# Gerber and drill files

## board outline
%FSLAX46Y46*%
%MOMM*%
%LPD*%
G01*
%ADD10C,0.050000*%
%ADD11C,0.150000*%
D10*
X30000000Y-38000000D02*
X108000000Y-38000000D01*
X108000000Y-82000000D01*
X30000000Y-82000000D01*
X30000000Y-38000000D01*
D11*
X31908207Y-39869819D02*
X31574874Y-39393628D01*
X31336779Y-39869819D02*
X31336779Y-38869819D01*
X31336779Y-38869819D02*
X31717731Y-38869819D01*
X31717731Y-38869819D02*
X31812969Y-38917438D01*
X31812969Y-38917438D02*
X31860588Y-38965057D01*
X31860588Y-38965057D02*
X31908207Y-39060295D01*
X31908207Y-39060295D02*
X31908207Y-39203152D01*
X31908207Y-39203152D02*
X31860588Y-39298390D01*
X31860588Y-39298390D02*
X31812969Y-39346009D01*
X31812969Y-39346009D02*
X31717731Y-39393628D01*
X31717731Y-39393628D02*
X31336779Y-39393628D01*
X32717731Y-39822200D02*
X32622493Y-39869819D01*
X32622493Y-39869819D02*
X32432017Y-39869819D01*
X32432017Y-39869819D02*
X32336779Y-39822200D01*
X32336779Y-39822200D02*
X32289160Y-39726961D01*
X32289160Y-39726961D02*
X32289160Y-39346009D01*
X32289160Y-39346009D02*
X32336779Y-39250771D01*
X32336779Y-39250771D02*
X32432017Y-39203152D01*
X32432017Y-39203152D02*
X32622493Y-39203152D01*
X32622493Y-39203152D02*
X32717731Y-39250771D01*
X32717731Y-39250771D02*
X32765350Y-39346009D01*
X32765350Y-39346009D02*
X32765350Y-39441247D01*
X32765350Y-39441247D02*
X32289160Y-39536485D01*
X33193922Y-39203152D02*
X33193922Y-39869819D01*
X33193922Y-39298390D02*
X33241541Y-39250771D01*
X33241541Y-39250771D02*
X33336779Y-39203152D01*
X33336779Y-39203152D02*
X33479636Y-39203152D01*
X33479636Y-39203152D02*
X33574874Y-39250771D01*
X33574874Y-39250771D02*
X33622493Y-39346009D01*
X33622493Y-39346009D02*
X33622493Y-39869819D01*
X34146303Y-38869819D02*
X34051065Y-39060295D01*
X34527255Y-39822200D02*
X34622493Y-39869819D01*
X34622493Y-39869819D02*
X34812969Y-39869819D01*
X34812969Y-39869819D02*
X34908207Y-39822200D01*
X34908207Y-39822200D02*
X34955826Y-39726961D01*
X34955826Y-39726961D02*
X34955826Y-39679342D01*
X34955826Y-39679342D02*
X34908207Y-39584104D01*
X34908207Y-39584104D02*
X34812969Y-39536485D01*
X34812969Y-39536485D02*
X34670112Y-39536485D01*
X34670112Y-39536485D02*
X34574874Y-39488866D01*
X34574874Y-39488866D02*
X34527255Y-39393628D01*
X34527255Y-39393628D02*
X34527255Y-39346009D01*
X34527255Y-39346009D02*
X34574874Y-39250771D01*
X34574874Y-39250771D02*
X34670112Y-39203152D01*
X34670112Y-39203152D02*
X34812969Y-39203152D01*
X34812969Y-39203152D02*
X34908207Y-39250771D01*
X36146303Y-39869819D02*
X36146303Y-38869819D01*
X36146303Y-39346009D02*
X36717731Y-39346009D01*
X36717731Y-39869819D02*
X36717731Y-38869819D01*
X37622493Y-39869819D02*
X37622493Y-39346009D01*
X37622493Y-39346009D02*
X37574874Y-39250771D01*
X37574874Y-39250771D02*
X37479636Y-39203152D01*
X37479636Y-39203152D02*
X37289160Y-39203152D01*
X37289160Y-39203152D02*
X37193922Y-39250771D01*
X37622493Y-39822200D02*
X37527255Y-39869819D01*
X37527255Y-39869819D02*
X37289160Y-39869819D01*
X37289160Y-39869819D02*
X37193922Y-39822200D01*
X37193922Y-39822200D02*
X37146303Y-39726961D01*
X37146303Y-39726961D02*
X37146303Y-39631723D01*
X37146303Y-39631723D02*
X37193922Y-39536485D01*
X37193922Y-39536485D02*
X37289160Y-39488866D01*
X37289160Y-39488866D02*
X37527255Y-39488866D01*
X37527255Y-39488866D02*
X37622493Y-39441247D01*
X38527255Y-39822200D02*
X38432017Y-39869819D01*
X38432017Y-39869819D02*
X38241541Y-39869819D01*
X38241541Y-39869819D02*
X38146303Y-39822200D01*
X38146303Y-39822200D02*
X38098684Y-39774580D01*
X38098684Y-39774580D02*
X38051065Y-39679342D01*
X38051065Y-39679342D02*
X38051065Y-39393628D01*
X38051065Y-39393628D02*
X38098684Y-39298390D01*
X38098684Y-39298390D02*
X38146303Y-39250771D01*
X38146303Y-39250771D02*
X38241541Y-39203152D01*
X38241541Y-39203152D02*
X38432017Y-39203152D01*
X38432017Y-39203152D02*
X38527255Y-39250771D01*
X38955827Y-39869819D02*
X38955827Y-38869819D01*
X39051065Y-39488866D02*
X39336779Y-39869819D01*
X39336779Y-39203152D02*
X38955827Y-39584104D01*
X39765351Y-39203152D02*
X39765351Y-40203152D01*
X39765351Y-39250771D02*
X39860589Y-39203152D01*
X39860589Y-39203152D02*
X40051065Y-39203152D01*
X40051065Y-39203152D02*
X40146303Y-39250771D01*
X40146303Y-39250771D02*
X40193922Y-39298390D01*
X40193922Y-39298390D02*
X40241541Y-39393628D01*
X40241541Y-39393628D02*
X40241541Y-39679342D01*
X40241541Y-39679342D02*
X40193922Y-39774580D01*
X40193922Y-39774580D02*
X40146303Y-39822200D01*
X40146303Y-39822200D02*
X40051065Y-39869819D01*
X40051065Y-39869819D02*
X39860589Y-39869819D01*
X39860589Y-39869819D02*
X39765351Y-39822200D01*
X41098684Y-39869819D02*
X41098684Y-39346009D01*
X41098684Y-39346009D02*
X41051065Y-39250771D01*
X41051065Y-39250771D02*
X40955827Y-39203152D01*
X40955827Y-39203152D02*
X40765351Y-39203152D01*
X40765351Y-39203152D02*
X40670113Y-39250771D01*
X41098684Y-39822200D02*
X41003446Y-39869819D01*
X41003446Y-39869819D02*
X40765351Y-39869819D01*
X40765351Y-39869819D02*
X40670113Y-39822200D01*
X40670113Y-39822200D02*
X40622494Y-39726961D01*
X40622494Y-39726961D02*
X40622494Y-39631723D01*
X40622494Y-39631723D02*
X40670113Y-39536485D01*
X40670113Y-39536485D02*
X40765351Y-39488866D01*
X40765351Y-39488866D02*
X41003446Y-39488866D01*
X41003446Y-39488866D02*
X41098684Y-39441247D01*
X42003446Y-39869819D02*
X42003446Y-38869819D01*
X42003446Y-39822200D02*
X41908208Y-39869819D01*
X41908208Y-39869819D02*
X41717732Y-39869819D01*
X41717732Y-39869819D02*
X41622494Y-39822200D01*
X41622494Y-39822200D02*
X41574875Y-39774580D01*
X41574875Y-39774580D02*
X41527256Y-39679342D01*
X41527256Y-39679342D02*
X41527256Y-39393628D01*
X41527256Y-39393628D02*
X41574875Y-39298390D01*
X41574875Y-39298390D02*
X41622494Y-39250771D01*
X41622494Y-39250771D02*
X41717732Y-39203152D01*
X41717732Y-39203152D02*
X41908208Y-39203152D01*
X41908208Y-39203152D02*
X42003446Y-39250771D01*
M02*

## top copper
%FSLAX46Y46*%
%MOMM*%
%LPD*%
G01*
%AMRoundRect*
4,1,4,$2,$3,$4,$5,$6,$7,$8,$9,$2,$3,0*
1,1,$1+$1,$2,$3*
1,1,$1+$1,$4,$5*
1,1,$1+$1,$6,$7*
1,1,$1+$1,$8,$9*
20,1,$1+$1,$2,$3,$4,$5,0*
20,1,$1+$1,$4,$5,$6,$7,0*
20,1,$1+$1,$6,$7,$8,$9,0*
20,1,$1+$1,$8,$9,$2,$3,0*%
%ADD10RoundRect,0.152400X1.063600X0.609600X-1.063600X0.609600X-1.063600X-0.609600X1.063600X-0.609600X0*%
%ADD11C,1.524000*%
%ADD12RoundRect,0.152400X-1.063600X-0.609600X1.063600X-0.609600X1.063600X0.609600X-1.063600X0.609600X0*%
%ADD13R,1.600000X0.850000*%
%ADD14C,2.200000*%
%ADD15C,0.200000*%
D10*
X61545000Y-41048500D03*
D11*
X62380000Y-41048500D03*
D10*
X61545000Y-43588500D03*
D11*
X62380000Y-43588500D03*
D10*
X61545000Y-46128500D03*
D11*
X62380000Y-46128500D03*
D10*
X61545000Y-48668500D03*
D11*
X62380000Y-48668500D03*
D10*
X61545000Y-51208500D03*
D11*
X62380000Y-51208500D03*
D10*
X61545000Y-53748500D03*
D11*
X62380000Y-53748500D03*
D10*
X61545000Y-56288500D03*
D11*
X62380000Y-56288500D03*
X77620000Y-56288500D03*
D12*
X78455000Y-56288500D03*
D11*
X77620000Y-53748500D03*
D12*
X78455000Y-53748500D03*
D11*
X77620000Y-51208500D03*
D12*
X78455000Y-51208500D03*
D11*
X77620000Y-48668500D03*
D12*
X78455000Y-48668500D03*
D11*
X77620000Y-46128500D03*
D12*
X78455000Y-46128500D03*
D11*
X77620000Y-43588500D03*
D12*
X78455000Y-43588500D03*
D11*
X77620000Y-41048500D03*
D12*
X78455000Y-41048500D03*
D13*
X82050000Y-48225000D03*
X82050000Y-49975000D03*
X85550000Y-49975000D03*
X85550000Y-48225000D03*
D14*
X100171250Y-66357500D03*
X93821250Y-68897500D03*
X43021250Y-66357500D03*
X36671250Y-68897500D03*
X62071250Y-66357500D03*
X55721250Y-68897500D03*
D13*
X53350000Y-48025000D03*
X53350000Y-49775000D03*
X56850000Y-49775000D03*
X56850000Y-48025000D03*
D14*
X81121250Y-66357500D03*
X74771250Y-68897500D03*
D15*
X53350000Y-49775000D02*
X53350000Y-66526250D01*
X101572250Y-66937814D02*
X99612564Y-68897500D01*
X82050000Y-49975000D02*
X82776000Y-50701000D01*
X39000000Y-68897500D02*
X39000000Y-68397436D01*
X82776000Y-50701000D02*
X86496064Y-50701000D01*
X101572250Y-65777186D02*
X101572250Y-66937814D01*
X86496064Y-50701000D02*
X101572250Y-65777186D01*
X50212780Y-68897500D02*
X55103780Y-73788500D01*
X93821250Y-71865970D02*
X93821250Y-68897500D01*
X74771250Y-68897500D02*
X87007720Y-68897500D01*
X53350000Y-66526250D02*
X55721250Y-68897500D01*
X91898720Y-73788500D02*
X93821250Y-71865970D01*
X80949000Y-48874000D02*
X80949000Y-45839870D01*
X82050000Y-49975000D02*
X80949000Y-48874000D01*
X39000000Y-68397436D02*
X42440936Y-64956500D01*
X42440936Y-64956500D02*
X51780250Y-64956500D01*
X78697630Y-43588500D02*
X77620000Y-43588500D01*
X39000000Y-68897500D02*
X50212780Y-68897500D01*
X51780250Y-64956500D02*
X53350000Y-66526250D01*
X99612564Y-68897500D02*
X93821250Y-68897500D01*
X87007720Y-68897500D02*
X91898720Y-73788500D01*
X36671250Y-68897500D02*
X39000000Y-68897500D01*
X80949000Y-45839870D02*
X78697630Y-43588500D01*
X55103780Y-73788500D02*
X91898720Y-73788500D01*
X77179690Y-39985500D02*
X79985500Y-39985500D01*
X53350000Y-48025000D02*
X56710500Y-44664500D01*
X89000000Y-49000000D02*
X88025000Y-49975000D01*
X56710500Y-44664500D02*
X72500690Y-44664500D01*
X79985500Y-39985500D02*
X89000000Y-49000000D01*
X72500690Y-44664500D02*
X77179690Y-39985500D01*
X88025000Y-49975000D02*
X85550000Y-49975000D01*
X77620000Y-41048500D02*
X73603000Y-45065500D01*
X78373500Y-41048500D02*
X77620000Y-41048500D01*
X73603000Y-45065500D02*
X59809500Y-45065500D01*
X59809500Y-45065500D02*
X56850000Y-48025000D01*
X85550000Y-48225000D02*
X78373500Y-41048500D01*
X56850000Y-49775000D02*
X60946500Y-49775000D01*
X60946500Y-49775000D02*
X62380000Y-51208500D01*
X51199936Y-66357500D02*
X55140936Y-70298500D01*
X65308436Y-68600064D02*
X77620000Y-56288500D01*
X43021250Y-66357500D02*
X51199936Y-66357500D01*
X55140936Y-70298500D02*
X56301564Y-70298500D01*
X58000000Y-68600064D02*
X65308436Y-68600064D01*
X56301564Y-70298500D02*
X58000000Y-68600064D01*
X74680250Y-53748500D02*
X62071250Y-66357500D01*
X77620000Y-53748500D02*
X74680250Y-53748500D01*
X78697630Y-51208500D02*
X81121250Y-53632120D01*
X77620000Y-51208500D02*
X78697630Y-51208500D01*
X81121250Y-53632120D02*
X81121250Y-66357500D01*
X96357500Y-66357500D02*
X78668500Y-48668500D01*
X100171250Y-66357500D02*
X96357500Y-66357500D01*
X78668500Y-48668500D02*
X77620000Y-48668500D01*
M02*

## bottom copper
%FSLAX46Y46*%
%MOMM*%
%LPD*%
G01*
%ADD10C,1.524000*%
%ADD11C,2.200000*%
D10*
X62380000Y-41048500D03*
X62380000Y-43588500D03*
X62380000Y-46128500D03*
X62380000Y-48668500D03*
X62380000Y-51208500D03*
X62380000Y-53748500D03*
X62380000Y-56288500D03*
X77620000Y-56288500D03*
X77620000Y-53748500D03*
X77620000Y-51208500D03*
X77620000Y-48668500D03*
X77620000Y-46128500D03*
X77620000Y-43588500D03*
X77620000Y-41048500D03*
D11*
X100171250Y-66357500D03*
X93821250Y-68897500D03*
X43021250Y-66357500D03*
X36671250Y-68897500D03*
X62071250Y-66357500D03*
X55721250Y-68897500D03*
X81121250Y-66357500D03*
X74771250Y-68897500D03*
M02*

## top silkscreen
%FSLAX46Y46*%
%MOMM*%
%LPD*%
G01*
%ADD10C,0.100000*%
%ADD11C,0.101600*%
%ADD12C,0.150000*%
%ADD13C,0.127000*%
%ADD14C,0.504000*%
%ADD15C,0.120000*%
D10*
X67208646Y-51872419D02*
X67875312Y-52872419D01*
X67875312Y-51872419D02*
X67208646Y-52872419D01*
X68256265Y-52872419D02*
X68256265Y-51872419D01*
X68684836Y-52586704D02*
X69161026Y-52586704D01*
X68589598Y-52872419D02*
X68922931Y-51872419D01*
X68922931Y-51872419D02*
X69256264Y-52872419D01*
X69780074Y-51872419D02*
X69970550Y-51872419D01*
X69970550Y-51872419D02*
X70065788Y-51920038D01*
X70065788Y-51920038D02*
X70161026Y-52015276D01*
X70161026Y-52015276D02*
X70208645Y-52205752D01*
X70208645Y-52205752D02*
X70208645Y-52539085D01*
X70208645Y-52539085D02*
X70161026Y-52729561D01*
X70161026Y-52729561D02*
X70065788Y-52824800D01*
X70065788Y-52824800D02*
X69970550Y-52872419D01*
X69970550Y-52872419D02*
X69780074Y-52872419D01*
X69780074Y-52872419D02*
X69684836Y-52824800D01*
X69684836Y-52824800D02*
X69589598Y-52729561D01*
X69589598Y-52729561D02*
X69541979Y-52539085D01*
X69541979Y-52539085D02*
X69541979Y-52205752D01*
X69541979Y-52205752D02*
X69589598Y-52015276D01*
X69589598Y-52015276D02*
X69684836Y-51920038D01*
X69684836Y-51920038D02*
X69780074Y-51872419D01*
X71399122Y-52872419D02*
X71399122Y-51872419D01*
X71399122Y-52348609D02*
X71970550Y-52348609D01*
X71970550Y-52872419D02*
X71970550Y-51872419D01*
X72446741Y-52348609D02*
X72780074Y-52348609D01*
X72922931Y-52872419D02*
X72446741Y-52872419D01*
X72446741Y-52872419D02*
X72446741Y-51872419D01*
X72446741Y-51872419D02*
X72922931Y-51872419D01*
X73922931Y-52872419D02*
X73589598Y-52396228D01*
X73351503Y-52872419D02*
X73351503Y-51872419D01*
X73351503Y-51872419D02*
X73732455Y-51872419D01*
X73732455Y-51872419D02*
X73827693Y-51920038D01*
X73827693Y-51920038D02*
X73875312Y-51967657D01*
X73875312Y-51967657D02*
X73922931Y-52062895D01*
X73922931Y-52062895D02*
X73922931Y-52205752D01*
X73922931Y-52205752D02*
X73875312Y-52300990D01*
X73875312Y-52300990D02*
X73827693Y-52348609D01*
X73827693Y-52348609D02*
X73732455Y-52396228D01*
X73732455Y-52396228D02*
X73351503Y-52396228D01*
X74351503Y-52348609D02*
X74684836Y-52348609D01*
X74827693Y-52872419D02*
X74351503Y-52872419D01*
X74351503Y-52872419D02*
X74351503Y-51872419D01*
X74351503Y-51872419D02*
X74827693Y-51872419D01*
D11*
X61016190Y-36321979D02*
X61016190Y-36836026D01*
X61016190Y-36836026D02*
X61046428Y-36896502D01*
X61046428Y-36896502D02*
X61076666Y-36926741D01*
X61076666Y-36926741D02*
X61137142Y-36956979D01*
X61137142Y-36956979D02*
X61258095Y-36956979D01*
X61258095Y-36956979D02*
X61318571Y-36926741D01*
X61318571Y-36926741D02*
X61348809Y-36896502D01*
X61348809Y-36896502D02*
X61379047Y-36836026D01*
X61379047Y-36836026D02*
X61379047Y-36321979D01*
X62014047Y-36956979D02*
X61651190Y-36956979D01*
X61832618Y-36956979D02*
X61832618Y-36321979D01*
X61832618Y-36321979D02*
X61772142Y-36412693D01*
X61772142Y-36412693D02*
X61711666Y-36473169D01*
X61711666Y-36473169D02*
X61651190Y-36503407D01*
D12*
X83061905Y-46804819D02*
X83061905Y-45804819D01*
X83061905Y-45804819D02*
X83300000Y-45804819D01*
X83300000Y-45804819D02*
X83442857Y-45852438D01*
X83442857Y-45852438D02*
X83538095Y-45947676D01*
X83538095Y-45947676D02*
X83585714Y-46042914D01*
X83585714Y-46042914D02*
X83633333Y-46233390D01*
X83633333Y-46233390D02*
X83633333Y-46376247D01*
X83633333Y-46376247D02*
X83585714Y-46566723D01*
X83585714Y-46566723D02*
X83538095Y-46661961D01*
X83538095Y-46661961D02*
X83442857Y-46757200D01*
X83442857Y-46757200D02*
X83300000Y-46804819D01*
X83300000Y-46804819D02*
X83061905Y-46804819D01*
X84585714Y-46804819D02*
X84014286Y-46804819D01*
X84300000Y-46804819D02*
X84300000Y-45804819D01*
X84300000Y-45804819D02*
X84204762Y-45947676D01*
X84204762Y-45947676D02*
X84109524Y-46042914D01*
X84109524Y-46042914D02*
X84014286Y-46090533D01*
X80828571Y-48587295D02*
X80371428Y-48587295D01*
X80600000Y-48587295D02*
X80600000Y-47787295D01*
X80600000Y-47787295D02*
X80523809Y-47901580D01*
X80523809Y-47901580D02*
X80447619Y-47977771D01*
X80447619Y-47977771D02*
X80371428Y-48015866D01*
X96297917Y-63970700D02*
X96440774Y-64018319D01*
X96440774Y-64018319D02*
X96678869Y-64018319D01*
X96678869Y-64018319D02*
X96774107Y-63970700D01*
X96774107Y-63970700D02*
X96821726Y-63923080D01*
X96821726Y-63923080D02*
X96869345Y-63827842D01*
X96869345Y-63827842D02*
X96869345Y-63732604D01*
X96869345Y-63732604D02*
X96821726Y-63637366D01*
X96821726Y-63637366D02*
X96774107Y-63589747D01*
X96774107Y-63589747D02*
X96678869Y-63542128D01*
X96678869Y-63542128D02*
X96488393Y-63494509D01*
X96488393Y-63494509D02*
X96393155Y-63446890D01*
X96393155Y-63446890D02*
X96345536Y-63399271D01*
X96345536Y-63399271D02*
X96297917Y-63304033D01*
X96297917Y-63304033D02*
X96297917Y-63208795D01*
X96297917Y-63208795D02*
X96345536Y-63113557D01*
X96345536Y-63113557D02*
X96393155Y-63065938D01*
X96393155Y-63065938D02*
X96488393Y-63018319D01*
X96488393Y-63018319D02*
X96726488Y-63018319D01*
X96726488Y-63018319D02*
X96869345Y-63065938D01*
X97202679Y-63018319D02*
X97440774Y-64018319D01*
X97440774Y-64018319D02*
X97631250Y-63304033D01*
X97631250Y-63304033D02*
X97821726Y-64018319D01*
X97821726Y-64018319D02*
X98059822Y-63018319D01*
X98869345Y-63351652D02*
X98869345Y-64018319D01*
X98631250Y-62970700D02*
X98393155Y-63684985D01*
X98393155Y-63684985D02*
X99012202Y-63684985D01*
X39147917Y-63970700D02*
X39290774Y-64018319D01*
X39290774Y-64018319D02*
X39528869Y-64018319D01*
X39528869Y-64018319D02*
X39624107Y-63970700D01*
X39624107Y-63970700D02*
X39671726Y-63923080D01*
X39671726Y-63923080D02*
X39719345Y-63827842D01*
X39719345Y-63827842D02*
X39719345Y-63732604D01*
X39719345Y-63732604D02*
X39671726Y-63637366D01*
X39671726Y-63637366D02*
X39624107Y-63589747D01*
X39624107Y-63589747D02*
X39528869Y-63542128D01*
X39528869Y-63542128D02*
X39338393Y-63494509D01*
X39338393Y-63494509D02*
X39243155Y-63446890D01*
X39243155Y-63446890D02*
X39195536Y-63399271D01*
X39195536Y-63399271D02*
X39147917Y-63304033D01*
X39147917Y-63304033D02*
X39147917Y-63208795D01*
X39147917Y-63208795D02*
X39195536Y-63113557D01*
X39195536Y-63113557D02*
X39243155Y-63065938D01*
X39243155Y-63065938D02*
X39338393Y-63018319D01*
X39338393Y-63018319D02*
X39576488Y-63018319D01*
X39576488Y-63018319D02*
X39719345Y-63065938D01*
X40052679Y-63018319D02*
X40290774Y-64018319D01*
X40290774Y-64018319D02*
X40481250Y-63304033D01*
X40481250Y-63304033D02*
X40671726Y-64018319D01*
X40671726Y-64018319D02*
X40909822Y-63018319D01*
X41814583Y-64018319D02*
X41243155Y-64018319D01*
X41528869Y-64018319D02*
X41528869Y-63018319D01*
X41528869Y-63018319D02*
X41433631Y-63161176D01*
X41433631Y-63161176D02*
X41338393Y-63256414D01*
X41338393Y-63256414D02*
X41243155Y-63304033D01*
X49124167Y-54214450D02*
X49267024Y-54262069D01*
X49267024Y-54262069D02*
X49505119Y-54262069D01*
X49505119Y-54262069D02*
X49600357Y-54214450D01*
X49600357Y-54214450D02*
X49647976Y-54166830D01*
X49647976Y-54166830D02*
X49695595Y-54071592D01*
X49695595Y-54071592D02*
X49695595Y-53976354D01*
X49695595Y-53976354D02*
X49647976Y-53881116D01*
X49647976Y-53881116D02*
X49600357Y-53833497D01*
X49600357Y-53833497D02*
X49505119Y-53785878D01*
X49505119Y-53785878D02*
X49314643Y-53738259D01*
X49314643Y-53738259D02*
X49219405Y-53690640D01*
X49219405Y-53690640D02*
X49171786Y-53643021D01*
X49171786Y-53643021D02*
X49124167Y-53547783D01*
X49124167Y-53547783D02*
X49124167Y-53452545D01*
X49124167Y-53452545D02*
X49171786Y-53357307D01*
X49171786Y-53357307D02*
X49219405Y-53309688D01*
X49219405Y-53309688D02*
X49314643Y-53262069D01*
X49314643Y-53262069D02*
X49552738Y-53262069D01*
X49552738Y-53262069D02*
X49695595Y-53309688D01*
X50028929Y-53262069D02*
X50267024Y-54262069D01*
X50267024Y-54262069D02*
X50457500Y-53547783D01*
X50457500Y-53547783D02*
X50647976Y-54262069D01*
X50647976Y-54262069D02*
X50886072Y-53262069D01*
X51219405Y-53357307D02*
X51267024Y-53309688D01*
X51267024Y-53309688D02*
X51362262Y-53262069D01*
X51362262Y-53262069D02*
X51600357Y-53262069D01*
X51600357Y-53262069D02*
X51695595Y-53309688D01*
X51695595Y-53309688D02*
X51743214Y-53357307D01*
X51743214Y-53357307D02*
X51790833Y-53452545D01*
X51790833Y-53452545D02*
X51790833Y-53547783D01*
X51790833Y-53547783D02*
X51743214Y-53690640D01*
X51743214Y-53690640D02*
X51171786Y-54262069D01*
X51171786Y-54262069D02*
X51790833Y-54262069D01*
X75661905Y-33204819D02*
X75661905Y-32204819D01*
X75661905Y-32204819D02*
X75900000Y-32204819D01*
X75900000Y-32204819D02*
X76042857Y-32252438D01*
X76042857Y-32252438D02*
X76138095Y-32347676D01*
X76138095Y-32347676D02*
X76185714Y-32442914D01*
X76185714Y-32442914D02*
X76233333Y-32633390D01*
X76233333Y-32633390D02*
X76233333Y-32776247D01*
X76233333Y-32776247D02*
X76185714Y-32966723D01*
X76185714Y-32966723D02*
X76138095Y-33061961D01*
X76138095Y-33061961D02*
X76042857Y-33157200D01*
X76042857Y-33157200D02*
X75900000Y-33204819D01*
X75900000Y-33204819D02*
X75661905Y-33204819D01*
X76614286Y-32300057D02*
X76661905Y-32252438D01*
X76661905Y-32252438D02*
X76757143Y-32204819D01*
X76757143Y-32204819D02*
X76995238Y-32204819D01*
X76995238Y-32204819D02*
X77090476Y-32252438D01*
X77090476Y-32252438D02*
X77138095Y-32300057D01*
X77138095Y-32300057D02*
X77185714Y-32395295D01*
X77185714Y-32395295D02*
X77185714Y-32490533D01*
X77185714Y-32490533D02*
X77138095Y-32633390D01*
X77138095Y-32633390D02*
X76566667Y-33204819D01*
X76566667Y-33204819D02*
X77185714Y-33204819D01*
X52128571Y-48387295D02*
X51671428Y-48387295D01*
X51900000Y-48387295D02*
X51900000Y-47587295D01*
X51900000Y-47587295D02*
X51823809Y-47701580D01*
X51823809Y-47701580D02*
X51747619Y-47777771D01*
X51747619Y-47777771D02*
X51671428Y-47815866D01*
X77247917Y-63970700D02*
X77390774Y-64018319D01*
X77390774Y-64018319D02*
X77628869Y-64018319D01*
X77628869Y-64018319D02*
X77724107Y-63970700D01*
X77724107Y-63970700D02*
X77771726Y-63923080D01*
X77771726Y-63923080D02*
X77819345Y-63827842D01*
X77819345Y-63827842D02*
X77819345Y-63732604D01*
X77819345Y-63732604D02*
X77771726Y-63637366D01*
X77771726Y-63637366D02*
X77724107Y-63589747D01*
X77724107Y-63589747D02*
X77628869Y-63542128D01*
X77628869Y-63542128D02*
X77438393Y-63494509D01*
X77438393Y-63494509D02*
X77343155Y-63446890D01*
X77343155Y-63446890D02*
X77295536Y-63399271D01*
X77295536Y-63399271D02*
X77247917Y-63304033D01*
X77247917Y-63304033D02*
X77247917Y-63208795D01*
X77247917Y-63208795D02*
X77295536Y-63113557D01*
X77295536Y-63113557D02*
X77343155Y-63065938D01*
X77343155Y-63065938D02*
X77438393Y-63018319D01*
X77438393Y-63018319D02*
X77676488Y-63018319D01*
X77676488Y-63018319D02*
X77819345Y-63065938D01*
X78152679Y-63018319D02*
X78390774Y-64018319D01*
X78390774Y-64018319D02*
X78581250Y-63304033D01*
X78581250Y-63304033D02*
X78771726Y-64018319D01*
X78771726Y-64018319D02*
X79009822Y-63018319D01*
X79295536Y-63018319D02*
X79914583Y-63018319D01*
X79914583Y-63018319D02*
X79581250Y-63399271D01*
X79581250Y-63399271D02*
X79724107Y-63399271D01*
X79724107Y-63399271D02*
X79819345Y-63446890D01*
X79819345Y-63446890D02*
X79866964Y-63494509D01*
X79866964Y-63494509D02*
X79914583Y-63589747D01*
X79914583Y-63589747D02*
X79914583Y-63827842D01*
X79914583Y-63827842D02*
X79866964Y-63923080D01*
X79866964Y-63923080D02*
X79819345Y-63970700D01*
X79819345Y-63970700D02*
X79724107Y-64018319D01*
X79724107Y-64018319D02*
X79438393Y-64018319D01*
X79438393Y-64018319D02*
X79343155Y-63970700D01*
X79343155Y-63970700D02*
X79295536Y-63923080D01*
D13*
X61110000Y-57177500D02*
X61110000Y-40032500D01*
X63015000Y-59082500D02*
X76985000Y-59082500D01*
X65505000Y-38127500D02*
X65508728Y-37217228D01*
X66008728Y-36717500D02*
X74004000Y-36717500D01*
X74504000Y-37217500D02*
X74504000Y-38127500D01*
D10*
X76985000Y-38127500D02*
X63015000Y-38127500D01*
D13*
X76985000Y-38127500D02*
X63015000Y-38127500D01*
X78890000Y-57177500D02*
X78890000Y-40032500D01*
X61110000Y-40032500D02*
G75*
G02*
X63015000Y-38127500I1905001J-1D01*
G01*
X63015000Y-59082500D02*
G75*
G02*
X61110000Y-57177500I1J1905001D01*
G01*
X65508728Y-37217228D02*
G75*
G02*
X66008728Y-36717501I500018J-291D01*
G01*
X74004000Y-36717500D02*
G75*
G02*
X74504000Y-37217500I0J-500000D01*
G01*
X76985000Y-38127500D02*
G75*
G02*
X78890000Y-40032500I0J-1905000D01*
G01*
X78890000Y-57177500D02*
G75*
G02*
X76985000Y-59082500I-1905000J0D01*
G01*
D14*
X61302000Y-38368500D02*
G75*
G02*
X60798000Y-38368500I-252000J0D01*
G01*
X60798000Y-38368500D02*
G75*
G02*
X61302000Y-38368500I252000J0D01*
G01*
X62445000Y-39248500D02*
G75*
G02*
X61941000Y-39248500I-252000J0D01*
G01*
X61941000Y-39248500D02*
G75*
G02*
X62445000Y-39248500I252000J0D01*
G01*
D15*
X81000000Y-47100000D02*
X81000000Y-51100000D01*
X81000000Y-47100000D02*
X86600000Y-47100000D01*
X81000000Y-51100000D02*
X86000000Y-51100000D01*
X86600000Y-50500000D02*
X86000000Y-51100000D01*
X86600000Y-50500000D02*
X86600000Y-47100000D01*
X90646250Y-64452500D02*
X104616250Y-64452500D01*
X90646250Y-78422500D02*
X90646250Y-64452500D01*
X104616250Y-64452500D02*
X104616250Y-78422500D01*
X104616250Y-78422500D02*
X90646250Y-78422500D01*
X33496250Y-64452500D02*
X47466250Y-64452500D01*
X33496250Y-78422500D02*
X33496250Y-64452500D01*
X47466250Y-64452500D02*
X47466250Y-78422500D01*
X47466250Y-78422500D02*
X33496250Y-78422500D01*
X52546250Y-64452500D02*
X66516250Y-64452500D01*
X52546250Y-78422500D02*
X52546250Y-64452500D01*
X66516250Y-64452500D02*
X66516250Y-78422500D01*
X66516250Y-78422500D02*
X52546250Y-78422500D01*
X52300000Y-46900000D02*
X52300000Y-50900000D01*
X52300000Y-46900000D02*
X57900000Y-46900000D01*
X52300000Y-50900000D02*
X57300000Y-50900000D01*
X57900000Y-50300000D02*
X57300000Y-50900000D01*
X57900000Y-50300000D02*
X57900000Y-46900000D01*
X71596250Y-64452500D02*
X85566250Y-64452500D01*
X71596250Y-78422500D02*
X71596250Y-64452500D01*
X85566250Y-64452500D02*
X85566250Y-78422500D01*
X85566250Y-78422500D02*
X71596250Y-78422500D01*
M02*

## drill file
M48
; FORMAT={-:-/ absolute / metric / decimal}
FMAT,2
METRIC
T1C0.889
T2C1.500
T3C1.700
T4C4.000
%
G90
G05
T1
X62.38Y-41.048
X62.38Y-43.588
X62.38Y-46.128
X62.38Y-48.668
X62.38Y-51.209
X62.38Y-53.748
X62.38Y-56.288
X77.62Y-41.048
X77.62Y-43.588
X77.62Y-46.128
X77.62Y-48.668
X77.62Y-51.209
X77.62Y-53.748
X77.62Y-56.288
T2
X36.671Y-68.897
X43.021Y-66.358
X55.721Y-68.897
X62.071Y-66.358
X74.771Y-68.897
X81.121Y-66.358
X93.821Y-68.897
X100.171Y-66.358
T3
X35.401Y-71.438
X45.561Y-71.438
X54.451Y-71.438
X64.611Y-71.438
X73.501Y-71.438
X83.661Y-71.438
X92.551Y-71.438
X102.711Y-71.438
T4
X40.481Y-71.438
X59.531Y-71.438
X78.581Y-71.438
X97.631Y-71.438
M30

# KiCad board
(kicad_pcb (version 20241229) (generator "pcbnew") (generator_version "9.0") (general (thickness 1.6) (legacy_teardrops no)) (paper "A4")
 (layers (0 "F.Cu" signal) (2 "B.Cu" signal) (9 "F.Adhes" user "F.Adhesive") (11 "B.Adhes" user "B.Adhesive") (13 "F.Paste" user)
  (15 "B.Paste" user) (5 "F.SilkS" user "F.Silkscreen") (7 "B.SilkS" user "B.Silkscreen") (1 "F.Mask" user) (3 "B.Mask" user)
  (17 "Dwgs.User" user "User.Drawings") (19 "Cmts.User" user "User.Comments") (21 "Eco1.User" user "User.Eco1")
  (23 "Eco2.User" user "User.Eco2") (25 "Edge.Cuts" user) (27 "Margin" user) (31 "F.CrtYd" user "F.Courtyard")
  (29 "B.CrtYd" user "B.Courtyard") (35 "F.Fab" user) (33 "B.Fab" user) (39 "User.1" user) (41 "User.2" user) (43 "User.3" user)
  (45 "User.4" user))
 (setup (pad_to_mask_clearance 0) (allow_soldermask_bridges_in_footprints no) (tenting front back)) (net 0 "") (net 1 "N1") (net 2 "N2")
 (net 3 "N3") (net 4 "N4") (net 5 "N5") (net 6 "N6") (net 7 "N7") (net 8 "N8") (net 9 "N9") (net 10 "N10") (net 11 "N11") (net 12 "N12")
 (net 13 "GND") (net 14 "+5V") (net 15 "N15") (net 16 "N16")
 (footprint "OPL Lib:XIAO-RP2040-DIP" (layer "F.Cu") (at 70 48.6685)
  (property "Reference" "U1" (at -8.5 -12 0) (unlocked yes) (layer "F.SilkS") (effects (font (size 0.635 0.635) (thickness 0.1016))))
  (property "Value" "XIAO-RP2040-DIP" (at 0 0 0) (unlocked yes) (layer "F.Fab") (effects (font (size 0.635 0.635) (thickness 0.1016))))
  (fp_line (start -8.89 8.509) (end -8.89 -8.636) (stroke (width 0.127) (type solid)) (layer "F.SilkS"))
  (fp_line (start -6.985 10.414) (end 6.985 10.414) (stroke (width 0.127) (type solid)) (layer "F.SilkS"))
  (fp_line (start -4.495 -10.541) (end -4.491272 -11.451272) (stroke (width 0.127) (type solid)) (layer "F.SilkS"))
  (fp_line (start -3.991272 -11.951) (end 4.004 -11.951) (stroke (width 0.127) (type solid)) (layer "F.SilkS"))
  (fp_line (start 4.504 -11.451) (end 4.504 -10.541) (stroke (width 0.127) (type solid)) (layer "F.SilkS"))
  (fp_line (start 6.985 -10.541) (end -6.985 -10.541) (stroke (width 0.1) (type solid)) (layer "F.SilkS"))
  (fp_line (start 6.985 -10.541) (end -6.985 -10.541) (stroke (width 0.127) (type solid)) (layer "F.SilkS"))
  (fp_line (start 8.89 8.509) (end 8.89 -8.636) (stroke (width 0.127) (type solid)) (layer "F.SilkS"))
  (fp_arc (start -8.89 -8.636) (mid -8.332038 -9.983038) (end -6.985 -10.541) (stroke (width 0.127) (type solid)) (layer "F.SilkS"))
  (fp_arc (start -6.985 10.414) (mid -8.332038 9.856038) (end -8.89 8.509) (stroke (width 0.127) (type solid)) (layer "F.SilkS"))
  (fp_arc (start -4.491272 -11.451272) (mid -4.344728 -11.80464) (end -3.991272 -11.951) (stroke (width 0.127) (type default))
   (layer "F.SilkS"))
  (fp_arc (start 4.004 -11.951) (mid 4.357553 -11.804553) (end 4.504 -11.451) (stroke (width 0.127) (type default)) (layer "F.SilkS"))
  (fp_arc (start 6.985 -10.541) (mid 8.332038 -9.983038) (end 8.89 -8.636) (stroke (width 0.127) (type solid)) (layer "F.SilkS"))
  (fp_arc (start 8.89 8.509) (mid 8.332038 9.856038) (end 6.985 10.414) (stroke (width 0.127) (type solid)) (layer "F.SilkS"))
  (fp_circle (center -8.95 -10.3) (end -8.95 -10.554) (stroke (width 0.5) (type solid)) (fill yes) (layer "F.SilkS"))
  (fp_circle (center -7.807 -9.42) (end -7.807 -9.674) (stroke (width 0.5) (type solid)) (fill yes) (layer "F.SilkS"))
  (pad "1" smd roundrect (at -8.455 -7.62 180) (size 2.432 1.524) (layers "F.Cu" "F.Mask") (roundrect_rratio 0.1) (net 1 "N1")
   (thermal_bridge_angle 45))
  (pad "1" thru_hole circle (at -7.62 -7.62 180) (size 1.524 1.524) (drill 0.889) (layers "*.Cu" "*.Mask") (remove_unused_layers no)
   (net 1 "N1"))
  (pad "2" smd roundrect (at -8.455 -5.08 180) (size 2.432 1.524) (layers "F.Cu" "F.Mask") (roundrect_rratio 0.1) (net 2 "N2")
   (thermal_bridge_angle 45))
  (pad "2" thru_hole circle (at -7.62 -5.08 180) (size 1.524 1.524) (drill 0.889) (layers "*.Cu" "*.Mask") (remove_unused_layers no)
   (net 2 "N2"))
  (pad "3" smd roundrect (at -8.455 -2.54 180) (size 2.432 1.524) (layers "F.Cu" "F.Mask") (roundrect_rratio 0.1) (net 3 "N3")
   (thermal_bridge_angle 45))
  (pad "3" thru_hole circle (at -7.62 -2.54 180) (size 1.524 1.524) (drill 0.889) (layers "*.Cu" "*.Mask") (remove_unused_layers no)
   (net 3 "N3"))
  (pad "4" smd roundrect (at -8.455 0 180) (size 2.432 1.524) (layers "F.Cu" "F.Mask") (roundrect_rratio 0.1) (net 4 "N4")
   (thermal_bridge_angle 45))
  (pad "4" thru_hole circle (at -7.62 0 180) (size 1.524 1.524) (drill 0.889) (layers "*.Cu" "*.Mask") (remove_unused_layers no)
   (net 4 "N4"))
  (pad "5" smd roundrect (at -8.455 2.54 180) (size 2.432 1.524) (layers "F.Cu" "F.Mask") (roundrect_rratio 0.1) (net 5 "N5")
   (thermal_bridge_angle 45))
  (pad "5" thru_hole circle (at -7.62 2.54 180) (size 1.524 1.524) (drill 0.889) (layers "*.Cu" "*.Mask") (remove_unused_layers no)
   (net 5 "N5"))
  (pad "6" smd roundrect (at -8.455 5.08 180) (size 2.432 1.524) (layers "F.Cu" "F.Mask") (roundrect_rratio 0.1) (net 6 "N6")
   (thermal_bridge_angle 45))
  (pad "6" thru_hole circle (at -7.62 5.08 180) (size 1.524 1.524) (drill 0.889) (layers "*.Cu" "*.Mask") (remove_unused_layers no)
   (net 6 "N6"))
  (pad "7" smd roundrect (at -8.455 7.62 180) (size 2.432 1.524) (layers "F.Cu" "F.Mask") (roundrect_rratio 0.1) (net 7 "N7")
   (thermal_bridge_angle 45))
  (pad "7" thru_hole circle (at -7.62 7.62 180) (size 1.524 1.524) (drill 0.889) (layers "*.Cu" "*.Mask") (remove_unused_layers no)
   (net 7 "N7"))
  (pad "8" thru_hole circle (at 7.62 7.62) (size 1.524 1.524) (drill 0.889) (layers "*.Cu" "*.Mask") (remove_unused_layers no) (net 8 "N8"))
  (pad "8" smd roundrect (at 8.455 7.62) (size 2.432 1.524) (layers "F.Cu" "F.Mask") (roundrect_rratio 0.1) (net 8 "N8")
   (thermal_bridge_angle 45))
  (pad "9" thru_hole circle (at 7.62 5.08) (size 1.524 1.524) (drill 0.889) (layers "*.Cu" "*.Mask") (remove_unused_layers no) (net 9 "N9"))
  (pad "9" smd roundrect (at 8.455 5.08) (size 2.432 1.524) (layers "F.Cu" "F.Mask") (roundrect_rratio 0.1) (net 9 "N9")
   (thermal_bridge_angle 45))
  (pad "10" thru_hole circle (at 7.62 2.54) (size 1.524 1.524) (drill 0.889) (layers "*.Cu" "*.Mask") (remove_unused_layers no)
   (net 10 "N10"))
  (pad "10" smd roundrect (at 8.455 2.54) (size 2.432 1.524) (layers "F.Cu" "F.Mask") (roundrect_rratio 0.1) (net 10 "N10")
   (thermal_bridge_angle 45))
  (pad "11" thru_hole circle (at 7.62 0) (size 1.524 1.524) (drill 0.889) (layers "*.Cu" "*.Mask") (remove_unused_layers no) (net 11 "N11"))
  (pad "11" smd roundrect (at 8.455 0) (size 2.432 1.524) (layers "F.Cu" "F.Mask") (roundrect_rratio 0.1) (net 11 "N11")
   (thermal_bridge_angle 45))
  (pad "12" thru_hole circle (at 7.62 -2.54) (size 1.524 1.524) (drill 0.889) (layers "*.Cu" "*.Mask") (remove_unused_layers no)
   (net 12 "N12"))
  (pad "12" smd roundrect (at 8.455 -2.54) (size 2.432 1.524) (layers "F.Cu" "F.Mask") (roundrect_rratio 0.1) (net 12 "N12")
   (thermal_bridge_angle 45))
  (pad "13" thru_hole circle (at 7.62 -5.08) (size 1.524 1.524) (drill 0.889) (layers "*.Cu" "*.Mask") (remove_unused_layers no)
   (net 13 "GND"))
  (pad "13" smd roundrect (at 8.455 -5.08) (size 2.432 1.524) (layers "F.Cu" "F.Mask") (roundrect_rratio 0.1) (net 13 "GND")
   (thermal_bridge_angle 45))
  (pad "14" thru_hole circle (at 7.62 -7.62) (size 1.524 1.524) (drill 0.889) (layers "*.Cu" "*.Mask") (remove_unused_layers no)
   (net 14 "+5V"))
  (pad "14" smd roundrect (at 8.455 -7.62) (size 2.432 1.524) (layers "F.Cu" "F.Mask") (roundrect_rratio 0.1) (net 14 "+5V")
   (thermal_bridge_angle 45)))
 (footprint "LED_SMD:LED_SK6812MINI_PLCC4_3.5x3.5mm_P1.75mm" (layer "F.Cu") (at 83.8 49.1)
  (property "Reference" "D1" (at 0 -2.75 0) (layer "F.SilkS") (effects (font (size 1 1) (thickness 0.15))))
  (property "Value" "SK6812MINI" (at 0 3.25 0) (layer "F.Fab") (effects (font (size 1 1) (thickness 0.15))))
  (fp_line (start -2.8 -2) (end -2.8 2) (stroke (width 0.12) (type default)) (layer "F.SilkS"))
  (fp_line (start -2.8 -2) (end 2.8 -2) (stroke (width 0.12) (type solid)) (layer "F.SilkS"))
  (fp_line (start -2.8 2) (end 2.2 2) (stroke (width 0.12) (type solid)) (layer "F.SilkS"))
  (fp_line (start 2.8 1.4) (end 2.2 2) (stroke (width 0.12) (type default)) (layer "F.SilkS"))
  (fp_line (start 2.8 1.4) (end 2.8 -2) (stroke (width 0.12) (type solid)) (layer "F.SilkS"))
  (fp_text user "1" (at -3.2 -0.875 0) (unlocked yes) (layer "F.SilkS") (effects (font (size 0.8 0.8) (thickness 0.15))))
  (pad "1" smd rect (at -1.75 -0.875) (size 1.6 0.85) (layers "F.Cu" "F.Mask" "F.Paste") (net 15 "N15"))
  (pad "2" smd rect (at -1.75 0.875) (size 1.6 0.85) (layers "F.Cu" "F.Mask" "F.Paste") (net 13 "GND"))
  (pad "3" smd rect (at 1.75 0.875) (size 1.6 0.85) (layers "F.Cu" "F.Mask" "F.Paste") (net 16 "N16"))
  (pad "4" smd rect (at 1.75 -0.875) (size 1.6 0.85) (layers "F.Cu" "F.Mask" "F.Paste") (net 14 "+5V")))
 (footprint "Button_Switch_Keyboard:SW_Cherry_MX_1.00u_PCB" (layer "F.Cu") (at 100.17125 66.3575)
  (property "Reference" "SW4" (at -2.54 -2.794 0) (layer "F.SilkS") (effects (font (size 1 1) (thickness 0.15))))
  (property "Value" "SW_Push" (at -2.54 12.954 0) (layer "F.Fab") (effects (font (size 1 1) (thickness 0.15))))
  (fp_line (start -9.525 -1.905) (end 4.445 -1.905) (stroke (width 0.12) (type solid)) (layer "F.SilkS"))
  (fp_line (start -9.525 12.065) (end -9.525 -1.905) (stroke (width 0.12) (type solid)) (layer "F.SilkS"))
  (fp_line (start 4.445 -1.905) (end 4.445 12.065) (stroke (width 0.12) (type solid)) (layer "F.SilkS"))
  (fp_line (start 4.445 12.065) (end -9.525 12.065) (stroke (width 0.12) (type solid)) (layer "F.SilkS"))
  (pad "" np_thru_hole circle (at -7.62 5.08) (size 1.7 1.7) (drill 1.7) (layers "*.Cu" "*.Mask"))
  (pad "" np_thru_hole circle (at -2.54 5.08) (size 4 4) (drill 4) (layers "*.Cu" "*.Mask"))
  (pad "" np_thru_hole circle (at 2.54 5.08) (size 1.7 1.7) (drill 1.7) (layers "*.Cu" "*.Mask"))
  (pad "1" thru_hole circle (at 0 0) (size 2.2 2.2) (drill 1.5) (layers "*.Cu" "*.Mask") (remove_unused_layers no) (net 11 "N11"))
  (pad "2" thru_hole circle (at -6.35 2.54) (size 2.2 2.2) (drill 1.5) (layers "*.Cu" "*.Mask") (remove_unused_layers no) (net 13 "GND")))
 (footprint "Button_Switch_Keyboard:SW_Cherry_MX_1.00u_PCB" (layer "F.Cu") (at 43.02125 66.3575)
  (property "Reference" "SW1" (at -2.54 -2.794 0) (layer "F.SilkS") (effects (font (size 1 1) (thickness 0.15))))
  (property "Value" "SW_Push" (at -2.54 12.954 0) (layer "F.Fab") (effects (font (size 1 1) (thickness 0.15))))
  (fp_line (start -9.525 -1.905) (end 4.445 -1.905) (stroke (width 0.12) (type solid)) (layer "F.SilkS"))
  (fp_line (start -9.525 12.065) (end -9.525 -1.905) (stroke (width 0.12) (type solid)) (layer "F.SilkS"))
  (fp_line (start 4.445 -1.905) (end 4.445 12.065) (stroke (width 0.12) (type solid)) (layer "F.SilkS"))
  (fp_line (start 4.445 12.065) (end -9.525 12.065) (stroke (width 0.12) (type solid)) (layer "F.SilkS"))
  (pad "" np_thru_hole circle (at -7.62 5.08) (size 1.7 1.7) (drill 1.7) (layers "*.Cu" "*.Mask"))
  (pad "" np_thru_hole circle (at -2.54 5.08) (size 4 4) (drill 4) (layers "*.Cu" "*.Mask"))
  (pad "" np_thru_hole circle (at 2.54 5.08) (size 1.7 1.7) (drill 1.7) (layers "*.Cu" "*.Mask"))
  (pad "1" thru_hole circle (at 0 0) (size 2.2 2.2) (drill 1.5) (layers "*.Cu" "*.Mask") (remove_unused_layers no) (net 8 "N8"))
  (pad "2" thru_hole circle (at -6.35 2.54) (size 2.2 2.2) (drill 1.5) (layers "*.Cu" "*.Mask") (remove_unused_layers no) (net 13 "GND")))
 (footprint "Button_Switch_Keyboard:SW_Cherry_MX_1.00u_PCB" (layer "F.Cu") (at 62.07125 66.3575)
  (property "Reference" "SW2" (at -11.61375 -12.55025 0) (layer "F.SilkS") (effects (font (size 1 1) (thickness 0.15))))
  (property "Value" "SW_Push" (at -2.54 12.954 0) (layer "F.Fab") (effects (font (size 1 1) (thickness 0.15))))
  (fp_line (start -9.525 -1.905) (end 4.445 -1.905) (stroke (width 0.12) (type solid)) (layer "F.SilkS"))
  (fp_line (start -9.525 12.065) (end -9.525 -1.905) (stroke (width 0.12) (type solid)) (layer "F.SilkS"))
  (fp_line (start 4.445 -1.905) (end 4.445 12.065) (stroke (width 0.12) (type solid)) (layer "F.SilkS"))
  (fp_line (start 4.445 12.065) (end -9.525 12.065) (stroke (width 0.12) (type solid)) (layer "F.SilkS"))
  (pad "" np_thru_hole circle (at -7.62 5.08) (size 1.7 1.7) (drill 1.7) (layers "*.Cu" "*.Mask"))
  (pad "" np_thru_hole circle (at -2.54 5.08) (size 4 4) (drill 4) (layers "*.Cu" "*.Mask"))
  (pad "" np_thru_hole circle (at 2.54 5.08) (size 1.7 1.7) (drill 1.7) (layers "*.Cu" "*.Mask"))
  (pad "1" thru_hole circle (at 0 0) (size 2.2 2.2) (drill 1.5) (layers "*.Cu" "*.Mask") (remove_unused_layers no) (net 9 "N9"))
  (pad "2" thru_hole circle (at -6.35 2.54) (size 2.2 2.2) (drill 1.5) (layers "*.Cu" "*.Mask") (remove_unused_layers no) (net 13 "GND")))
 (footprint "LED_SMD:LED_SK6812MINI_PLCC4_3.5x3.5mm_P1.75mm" (layer "F.Cu") (at 55.1 48.9)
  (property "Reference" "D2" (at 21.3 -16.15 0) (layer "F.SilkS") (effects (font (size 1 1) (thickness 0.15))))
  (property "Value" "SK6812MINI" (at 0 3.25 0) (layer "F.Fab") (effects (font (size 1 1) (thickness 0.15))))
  (fp_line (start -2.8 -2) (end -2.8 2) (stroke (width 0.12) (type default)) (layer "F.SilkS"))
  (fp_line (start -2.8 -2) (end 2.8 -2) (stroke (width 0.12) (type solid)) (layer "F.SilkS"))
  (fp_line (start -2.8 2) (end 2.2 2) (stroke (width 0.12) (type solid)) (layer "F.SilkS"))
  (fp_line (start 2.8 1.4) (end 2.2 2) (stroke (width 0.12) (type default)) (layer "F.SilkS"))
  (fp_line (start 2.8 1.4) (end 2.8 -2) (stroke (width 0.12) (type solid)) (layer "F.SilkS"))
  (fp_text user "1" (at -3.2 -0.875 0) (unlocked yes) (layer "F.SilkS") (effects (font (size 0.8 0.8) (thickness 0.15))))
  (pad "1" smd rect (at -1.75 -0.875) (size 1.6 0.85) (layers "F.Cu" "F.Mask" "F.Paste") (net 16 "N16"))
  (pad "2" smd rect (at -1.75 0.875) (size 1.6 0.85) (layers "F.Cu" "F.Mask" "F.Paste") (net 13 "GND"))
  (pad "3" smd rect (at 1.75 0.875) (size 1.6 0.85) (layers "F.Cu" "F.Mask" "F.Paste") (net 5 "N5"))
  (pad "4" smd rect (at 1.75 -0.875) (size 1.6 0.85) (layers "F.Cu" "F.Mask" "F.Paste") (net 14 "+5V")))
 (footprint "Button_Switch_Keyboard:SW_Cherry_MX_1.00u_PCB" (layer "F.Cu") (at 81.12125 66.3575)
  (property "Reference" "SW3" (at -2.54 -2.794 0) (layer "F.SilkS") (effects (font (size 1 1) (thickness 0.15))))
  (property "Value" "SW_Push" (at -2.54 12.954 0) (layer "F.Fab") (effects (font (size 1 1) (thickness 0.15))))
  (fp_line (start -9.525 -1.905) (end 4.445 -1.905) (stroke (width 0.12) (type solid)) (layer "F.SilkS"))
  (fp_line (start -9.525 12.065) (end -9.525 -1.905) (stroke (width 0.12) (type solid)) (layer "F.SilkS"))
  (fp_line (start 4.445 -1.905) (end 4.445 12.065) (stroke (width 0.12) (type solid)) (layer "F.SilkS"))
  (fp_line (start 4.445 12.065) (end -9.525 12.065) (stroke (width 0.12) (type solid)) (layer "F.SilkS"))
  (pad "" np_thru_hole circle (at -7.62 5.08) (size 1.7 1.7) (drill 1.7) (layers "*.Cu" "*.Mask"))
  (pad "" np_thru_hole circle (at -2.54 5.08) (size 4 4) (drill 4) (layers "*.Cu" "*.Mask"))
  (pad "" np_thru_hole circle (at 2.54 5.08) (size 1.7 1.7) (drill 1.7) (layers "*.Cu" "*.Mask"))
  (pad "1" thru_hole circle (at 0 0) (size 2.2 2.2) (drill 1.5) (layers "*.Cu" "*.Mask") (remove_unused_layers no) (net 10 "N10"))
  (pad "2" thru_hole circle (at -6.35 2.54) (size 2.2 2.2) (drill 1.5) (layers "*.Cu" "*.Mask") (remove_unused_layers no) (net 13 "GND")))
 (gr_rect (start 30 38) (end 108 82) (stroke (width 0.05) (type default)) (fill no) (layer "Edge.Cuts"))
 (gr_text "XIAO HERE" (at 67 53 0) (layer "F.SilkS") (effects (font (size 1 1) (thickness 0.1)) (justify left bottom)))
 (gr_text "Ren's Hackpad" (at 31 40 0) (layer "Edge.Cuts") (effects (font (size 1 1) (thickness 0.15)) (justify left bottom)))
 (segment (start 53.35 49.775) (end 53.35 66.52625) (width 0.2) (layer "F.Cu") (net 13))
 (segment (start 101.57225 66.937814) (end 99.612564 68.8975) (width 0.2) (layer "F.Cu") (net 13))
 (segment (start 82.05 49.975) (end 82.776 50.701) (width 0.2) (layer "F.Cu") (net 13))
 (segment (start 39 68.8975) (end 39 68.397436) (width 0.2) (layer "F.Cu") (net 13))
 (segment (start 82.776 50.701) (end 86.496064 50.701) (width 0.2) (layer "F.Cu") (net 13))
 (segment (start 101.57225 65.777186) (end 101.57225 66.937814) (width 0.2) (layer "F.Cu") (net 13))
 (segment (start 86.496064 50.701) (end 101.57225 65.777186) (width 0.2) (layer "F.Cu") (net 13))
 (segment (start 50.21278 68.8975) (end 55.10378 73.7885) (width 0.2) (layer "F.Cu") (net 13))
 (segment (start 93.82125 71.86597) (end 93.82125 68.8975) (width 0.2) (layer "F.Cu") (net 13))
 (segment (start 74.77125 68.8975) (end 87.00772 68.8975) (width 0.2) (layer "F.Cu") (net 13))
 (segment (start 53.35 66.52625) (end 55.72125 68.8975) (width 0.2) (layer "F.Cu") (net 13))
 (segment (start 91.89872 73.7885) (end 93.82125 71.86597) (width 0.2) (layer "F.Cu") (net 13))
 (segment (start 80.949 48.874) (end 80.949 45.83987) (width 0.2) (layer "F.Cu") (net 13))
 (segment (start 82.05 49.975) (end 80.949 48.874) (width 0.2) (layer "F.Cu") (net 13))
 (segment (start 39 68.397436) (end 42.440936 64.9565) (width 0.2) (layer "F.Cu") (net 13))
 (segment (start 42.440936 64.9565) (end 51.78025 64.9565) (width 0.2) (layer "F.Cu") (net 13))
 (segment (start 78.69763 43.5885) (end 77.62 43.5885) (width 0.2) (layer "F.Cu") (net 13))
 (segment (start 39 68.8975) (end 50.21278 68.8975) (width 0.2) (layer "F.Cu") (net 13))
 (segment (start 51.78025 64.9565) (end 53.35 66.52625) (width 0.2) (layer "F.Cu") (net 13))
 (segment (start 99.612564 68.8975) (end 93.82125 68.8975) (width 0.2) (layer "F.Cu") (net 13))
 (segment (start 87.00772 68.8975) (end 91.89872 73.7885) (width 0.2) (layer "F.Cu") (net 13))
 (segment (start 36.67125 68.8975) (end 39 68.8975) (width 0.2) (layer "F.Cu") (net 13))
 (segment (start 80.949 45.83987) (end 78.69763 43.5885) (width 0.2) (layer "F.Cu") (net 13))
 (segment (start 55.10378 73.7885) (end 91.89872 73.7885) (width 0.2) (layer "F.Cu") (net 13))
 (segment (start 77.17969 39.9855) (end 79.9855 39.9855) (width 0.2) (layer "F.Cu") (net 16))
 (segment (start 53.35 48.025) (end 56.7105 44.6645) (width 0.2) (layer "F.Cu") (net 16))
 (segment (start 89 49) (end 88.025 49.975) (width 0.2) (layer "F.Cu") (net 16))
 (segment (start 56.7105 44.6645) (end 72.50069 44.6645) (width 0.2) (layer "F.Cu") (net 16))
 (segment (start 79.9855 39.9855) (end 89 49) (width 0.2) (layer "F.Cu") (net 16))
 (segment (start 72.50069 44.6645) (end 77.17969 39.9855) (width 0.2) (layer "F.Cu") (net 16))
 (segment (start 88.025 49.975) (end 85.55 49.975) (width 0.2) (layer "F.Cu") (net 16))
 (segment (start 77.62 41.0485) (end 73.603 45.0655) (width 0.2) (layer "F.Cu") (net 14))
 (segment (start 78.3735 41.0485) (end 77.62 41.0485) (width 0.2) (layer "F.Cu") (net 14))
 (segment (start 73.603 45.0655) (end 59.8095 45.0655) (width 0.2) (layer "F.Cu") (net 14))
 (segment (start 59.8095 45.0655) (end 56.85 48.025) (width 0.2) (layer "F.Cu") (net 14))
 (segment (start 85.55 48.225) (end 78.3735 41.0485) (width 0.2) (layer "F.Cu") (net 14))
 (segment (start 56.85 49.775) (end 60.9465 49.775) (width 0.2) (layer "F.Cu") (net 5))
 (segment (start 60.9465 49.775) (end 62.38 51.2085) (width 0.2) (layer "F.Cu") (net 5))
 (segment (start 51.199936 66.3575) (end 55.140936 70.2985) (width 0.2) (layer "F.Cu") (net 8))
 (segment (start 65.308436 68.600064) (end 77.62 56.2885) (width 0.2) (layer "F.Cu") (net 8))
 (segment (start 43.02125 66.3575) (end 51.199936 66.3575) (width 0.2) (layer "F.Cu") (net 8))
 (segment (start 55.140936 70.2985) (end 56.301564 70.2985) (width 0.2) (layer "F.Cu") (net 8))
 (segment (start 58 68.600064) (end 65.308436 68.600064) (width 0.2) (layer "F.Cu") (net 8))
 (segment (start 56.301564 70.2985) (end 58 68.600064) (width 0.2) (layer "F.Cu") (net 8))
 (segment (start 74.68025 53.7485) (end 62.07125 66.3575) (width 0.2) (layer "F.Cu") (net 9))
 (segment (start 77.62 53.7485) (end 74.68025 53.7485) (width 0.2) (layer "F.Cu") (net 9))
 (segment (start 78.69763 51.2085) (end 81.12125 53.63212) (width 0.2) (layer "F.Cu") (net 10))
 (segment (start 77.62 51.2085) (end 78.69763 51.2085) (width 0.2) (layer "F.Cu") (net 10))
 (segment (start 81.12125 53.63212) (end 81.12125 66.3575) (width 0.2) (layer "F.Cu") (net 10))
 (segment (start 96.3575 66.3575) (end 78.6685 48.6685) (width 0.2) (layer "F.Cu") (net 11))
 (segment (start 100.17125 66.3575) (end 96.3575 66.3575) (width 0.2) (layer "F.Cu") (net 11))
 (segment (start 78.6685 48.6685) (end 77.62 48.6685) (width 0.2) (layer "F.Cu") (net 11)))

